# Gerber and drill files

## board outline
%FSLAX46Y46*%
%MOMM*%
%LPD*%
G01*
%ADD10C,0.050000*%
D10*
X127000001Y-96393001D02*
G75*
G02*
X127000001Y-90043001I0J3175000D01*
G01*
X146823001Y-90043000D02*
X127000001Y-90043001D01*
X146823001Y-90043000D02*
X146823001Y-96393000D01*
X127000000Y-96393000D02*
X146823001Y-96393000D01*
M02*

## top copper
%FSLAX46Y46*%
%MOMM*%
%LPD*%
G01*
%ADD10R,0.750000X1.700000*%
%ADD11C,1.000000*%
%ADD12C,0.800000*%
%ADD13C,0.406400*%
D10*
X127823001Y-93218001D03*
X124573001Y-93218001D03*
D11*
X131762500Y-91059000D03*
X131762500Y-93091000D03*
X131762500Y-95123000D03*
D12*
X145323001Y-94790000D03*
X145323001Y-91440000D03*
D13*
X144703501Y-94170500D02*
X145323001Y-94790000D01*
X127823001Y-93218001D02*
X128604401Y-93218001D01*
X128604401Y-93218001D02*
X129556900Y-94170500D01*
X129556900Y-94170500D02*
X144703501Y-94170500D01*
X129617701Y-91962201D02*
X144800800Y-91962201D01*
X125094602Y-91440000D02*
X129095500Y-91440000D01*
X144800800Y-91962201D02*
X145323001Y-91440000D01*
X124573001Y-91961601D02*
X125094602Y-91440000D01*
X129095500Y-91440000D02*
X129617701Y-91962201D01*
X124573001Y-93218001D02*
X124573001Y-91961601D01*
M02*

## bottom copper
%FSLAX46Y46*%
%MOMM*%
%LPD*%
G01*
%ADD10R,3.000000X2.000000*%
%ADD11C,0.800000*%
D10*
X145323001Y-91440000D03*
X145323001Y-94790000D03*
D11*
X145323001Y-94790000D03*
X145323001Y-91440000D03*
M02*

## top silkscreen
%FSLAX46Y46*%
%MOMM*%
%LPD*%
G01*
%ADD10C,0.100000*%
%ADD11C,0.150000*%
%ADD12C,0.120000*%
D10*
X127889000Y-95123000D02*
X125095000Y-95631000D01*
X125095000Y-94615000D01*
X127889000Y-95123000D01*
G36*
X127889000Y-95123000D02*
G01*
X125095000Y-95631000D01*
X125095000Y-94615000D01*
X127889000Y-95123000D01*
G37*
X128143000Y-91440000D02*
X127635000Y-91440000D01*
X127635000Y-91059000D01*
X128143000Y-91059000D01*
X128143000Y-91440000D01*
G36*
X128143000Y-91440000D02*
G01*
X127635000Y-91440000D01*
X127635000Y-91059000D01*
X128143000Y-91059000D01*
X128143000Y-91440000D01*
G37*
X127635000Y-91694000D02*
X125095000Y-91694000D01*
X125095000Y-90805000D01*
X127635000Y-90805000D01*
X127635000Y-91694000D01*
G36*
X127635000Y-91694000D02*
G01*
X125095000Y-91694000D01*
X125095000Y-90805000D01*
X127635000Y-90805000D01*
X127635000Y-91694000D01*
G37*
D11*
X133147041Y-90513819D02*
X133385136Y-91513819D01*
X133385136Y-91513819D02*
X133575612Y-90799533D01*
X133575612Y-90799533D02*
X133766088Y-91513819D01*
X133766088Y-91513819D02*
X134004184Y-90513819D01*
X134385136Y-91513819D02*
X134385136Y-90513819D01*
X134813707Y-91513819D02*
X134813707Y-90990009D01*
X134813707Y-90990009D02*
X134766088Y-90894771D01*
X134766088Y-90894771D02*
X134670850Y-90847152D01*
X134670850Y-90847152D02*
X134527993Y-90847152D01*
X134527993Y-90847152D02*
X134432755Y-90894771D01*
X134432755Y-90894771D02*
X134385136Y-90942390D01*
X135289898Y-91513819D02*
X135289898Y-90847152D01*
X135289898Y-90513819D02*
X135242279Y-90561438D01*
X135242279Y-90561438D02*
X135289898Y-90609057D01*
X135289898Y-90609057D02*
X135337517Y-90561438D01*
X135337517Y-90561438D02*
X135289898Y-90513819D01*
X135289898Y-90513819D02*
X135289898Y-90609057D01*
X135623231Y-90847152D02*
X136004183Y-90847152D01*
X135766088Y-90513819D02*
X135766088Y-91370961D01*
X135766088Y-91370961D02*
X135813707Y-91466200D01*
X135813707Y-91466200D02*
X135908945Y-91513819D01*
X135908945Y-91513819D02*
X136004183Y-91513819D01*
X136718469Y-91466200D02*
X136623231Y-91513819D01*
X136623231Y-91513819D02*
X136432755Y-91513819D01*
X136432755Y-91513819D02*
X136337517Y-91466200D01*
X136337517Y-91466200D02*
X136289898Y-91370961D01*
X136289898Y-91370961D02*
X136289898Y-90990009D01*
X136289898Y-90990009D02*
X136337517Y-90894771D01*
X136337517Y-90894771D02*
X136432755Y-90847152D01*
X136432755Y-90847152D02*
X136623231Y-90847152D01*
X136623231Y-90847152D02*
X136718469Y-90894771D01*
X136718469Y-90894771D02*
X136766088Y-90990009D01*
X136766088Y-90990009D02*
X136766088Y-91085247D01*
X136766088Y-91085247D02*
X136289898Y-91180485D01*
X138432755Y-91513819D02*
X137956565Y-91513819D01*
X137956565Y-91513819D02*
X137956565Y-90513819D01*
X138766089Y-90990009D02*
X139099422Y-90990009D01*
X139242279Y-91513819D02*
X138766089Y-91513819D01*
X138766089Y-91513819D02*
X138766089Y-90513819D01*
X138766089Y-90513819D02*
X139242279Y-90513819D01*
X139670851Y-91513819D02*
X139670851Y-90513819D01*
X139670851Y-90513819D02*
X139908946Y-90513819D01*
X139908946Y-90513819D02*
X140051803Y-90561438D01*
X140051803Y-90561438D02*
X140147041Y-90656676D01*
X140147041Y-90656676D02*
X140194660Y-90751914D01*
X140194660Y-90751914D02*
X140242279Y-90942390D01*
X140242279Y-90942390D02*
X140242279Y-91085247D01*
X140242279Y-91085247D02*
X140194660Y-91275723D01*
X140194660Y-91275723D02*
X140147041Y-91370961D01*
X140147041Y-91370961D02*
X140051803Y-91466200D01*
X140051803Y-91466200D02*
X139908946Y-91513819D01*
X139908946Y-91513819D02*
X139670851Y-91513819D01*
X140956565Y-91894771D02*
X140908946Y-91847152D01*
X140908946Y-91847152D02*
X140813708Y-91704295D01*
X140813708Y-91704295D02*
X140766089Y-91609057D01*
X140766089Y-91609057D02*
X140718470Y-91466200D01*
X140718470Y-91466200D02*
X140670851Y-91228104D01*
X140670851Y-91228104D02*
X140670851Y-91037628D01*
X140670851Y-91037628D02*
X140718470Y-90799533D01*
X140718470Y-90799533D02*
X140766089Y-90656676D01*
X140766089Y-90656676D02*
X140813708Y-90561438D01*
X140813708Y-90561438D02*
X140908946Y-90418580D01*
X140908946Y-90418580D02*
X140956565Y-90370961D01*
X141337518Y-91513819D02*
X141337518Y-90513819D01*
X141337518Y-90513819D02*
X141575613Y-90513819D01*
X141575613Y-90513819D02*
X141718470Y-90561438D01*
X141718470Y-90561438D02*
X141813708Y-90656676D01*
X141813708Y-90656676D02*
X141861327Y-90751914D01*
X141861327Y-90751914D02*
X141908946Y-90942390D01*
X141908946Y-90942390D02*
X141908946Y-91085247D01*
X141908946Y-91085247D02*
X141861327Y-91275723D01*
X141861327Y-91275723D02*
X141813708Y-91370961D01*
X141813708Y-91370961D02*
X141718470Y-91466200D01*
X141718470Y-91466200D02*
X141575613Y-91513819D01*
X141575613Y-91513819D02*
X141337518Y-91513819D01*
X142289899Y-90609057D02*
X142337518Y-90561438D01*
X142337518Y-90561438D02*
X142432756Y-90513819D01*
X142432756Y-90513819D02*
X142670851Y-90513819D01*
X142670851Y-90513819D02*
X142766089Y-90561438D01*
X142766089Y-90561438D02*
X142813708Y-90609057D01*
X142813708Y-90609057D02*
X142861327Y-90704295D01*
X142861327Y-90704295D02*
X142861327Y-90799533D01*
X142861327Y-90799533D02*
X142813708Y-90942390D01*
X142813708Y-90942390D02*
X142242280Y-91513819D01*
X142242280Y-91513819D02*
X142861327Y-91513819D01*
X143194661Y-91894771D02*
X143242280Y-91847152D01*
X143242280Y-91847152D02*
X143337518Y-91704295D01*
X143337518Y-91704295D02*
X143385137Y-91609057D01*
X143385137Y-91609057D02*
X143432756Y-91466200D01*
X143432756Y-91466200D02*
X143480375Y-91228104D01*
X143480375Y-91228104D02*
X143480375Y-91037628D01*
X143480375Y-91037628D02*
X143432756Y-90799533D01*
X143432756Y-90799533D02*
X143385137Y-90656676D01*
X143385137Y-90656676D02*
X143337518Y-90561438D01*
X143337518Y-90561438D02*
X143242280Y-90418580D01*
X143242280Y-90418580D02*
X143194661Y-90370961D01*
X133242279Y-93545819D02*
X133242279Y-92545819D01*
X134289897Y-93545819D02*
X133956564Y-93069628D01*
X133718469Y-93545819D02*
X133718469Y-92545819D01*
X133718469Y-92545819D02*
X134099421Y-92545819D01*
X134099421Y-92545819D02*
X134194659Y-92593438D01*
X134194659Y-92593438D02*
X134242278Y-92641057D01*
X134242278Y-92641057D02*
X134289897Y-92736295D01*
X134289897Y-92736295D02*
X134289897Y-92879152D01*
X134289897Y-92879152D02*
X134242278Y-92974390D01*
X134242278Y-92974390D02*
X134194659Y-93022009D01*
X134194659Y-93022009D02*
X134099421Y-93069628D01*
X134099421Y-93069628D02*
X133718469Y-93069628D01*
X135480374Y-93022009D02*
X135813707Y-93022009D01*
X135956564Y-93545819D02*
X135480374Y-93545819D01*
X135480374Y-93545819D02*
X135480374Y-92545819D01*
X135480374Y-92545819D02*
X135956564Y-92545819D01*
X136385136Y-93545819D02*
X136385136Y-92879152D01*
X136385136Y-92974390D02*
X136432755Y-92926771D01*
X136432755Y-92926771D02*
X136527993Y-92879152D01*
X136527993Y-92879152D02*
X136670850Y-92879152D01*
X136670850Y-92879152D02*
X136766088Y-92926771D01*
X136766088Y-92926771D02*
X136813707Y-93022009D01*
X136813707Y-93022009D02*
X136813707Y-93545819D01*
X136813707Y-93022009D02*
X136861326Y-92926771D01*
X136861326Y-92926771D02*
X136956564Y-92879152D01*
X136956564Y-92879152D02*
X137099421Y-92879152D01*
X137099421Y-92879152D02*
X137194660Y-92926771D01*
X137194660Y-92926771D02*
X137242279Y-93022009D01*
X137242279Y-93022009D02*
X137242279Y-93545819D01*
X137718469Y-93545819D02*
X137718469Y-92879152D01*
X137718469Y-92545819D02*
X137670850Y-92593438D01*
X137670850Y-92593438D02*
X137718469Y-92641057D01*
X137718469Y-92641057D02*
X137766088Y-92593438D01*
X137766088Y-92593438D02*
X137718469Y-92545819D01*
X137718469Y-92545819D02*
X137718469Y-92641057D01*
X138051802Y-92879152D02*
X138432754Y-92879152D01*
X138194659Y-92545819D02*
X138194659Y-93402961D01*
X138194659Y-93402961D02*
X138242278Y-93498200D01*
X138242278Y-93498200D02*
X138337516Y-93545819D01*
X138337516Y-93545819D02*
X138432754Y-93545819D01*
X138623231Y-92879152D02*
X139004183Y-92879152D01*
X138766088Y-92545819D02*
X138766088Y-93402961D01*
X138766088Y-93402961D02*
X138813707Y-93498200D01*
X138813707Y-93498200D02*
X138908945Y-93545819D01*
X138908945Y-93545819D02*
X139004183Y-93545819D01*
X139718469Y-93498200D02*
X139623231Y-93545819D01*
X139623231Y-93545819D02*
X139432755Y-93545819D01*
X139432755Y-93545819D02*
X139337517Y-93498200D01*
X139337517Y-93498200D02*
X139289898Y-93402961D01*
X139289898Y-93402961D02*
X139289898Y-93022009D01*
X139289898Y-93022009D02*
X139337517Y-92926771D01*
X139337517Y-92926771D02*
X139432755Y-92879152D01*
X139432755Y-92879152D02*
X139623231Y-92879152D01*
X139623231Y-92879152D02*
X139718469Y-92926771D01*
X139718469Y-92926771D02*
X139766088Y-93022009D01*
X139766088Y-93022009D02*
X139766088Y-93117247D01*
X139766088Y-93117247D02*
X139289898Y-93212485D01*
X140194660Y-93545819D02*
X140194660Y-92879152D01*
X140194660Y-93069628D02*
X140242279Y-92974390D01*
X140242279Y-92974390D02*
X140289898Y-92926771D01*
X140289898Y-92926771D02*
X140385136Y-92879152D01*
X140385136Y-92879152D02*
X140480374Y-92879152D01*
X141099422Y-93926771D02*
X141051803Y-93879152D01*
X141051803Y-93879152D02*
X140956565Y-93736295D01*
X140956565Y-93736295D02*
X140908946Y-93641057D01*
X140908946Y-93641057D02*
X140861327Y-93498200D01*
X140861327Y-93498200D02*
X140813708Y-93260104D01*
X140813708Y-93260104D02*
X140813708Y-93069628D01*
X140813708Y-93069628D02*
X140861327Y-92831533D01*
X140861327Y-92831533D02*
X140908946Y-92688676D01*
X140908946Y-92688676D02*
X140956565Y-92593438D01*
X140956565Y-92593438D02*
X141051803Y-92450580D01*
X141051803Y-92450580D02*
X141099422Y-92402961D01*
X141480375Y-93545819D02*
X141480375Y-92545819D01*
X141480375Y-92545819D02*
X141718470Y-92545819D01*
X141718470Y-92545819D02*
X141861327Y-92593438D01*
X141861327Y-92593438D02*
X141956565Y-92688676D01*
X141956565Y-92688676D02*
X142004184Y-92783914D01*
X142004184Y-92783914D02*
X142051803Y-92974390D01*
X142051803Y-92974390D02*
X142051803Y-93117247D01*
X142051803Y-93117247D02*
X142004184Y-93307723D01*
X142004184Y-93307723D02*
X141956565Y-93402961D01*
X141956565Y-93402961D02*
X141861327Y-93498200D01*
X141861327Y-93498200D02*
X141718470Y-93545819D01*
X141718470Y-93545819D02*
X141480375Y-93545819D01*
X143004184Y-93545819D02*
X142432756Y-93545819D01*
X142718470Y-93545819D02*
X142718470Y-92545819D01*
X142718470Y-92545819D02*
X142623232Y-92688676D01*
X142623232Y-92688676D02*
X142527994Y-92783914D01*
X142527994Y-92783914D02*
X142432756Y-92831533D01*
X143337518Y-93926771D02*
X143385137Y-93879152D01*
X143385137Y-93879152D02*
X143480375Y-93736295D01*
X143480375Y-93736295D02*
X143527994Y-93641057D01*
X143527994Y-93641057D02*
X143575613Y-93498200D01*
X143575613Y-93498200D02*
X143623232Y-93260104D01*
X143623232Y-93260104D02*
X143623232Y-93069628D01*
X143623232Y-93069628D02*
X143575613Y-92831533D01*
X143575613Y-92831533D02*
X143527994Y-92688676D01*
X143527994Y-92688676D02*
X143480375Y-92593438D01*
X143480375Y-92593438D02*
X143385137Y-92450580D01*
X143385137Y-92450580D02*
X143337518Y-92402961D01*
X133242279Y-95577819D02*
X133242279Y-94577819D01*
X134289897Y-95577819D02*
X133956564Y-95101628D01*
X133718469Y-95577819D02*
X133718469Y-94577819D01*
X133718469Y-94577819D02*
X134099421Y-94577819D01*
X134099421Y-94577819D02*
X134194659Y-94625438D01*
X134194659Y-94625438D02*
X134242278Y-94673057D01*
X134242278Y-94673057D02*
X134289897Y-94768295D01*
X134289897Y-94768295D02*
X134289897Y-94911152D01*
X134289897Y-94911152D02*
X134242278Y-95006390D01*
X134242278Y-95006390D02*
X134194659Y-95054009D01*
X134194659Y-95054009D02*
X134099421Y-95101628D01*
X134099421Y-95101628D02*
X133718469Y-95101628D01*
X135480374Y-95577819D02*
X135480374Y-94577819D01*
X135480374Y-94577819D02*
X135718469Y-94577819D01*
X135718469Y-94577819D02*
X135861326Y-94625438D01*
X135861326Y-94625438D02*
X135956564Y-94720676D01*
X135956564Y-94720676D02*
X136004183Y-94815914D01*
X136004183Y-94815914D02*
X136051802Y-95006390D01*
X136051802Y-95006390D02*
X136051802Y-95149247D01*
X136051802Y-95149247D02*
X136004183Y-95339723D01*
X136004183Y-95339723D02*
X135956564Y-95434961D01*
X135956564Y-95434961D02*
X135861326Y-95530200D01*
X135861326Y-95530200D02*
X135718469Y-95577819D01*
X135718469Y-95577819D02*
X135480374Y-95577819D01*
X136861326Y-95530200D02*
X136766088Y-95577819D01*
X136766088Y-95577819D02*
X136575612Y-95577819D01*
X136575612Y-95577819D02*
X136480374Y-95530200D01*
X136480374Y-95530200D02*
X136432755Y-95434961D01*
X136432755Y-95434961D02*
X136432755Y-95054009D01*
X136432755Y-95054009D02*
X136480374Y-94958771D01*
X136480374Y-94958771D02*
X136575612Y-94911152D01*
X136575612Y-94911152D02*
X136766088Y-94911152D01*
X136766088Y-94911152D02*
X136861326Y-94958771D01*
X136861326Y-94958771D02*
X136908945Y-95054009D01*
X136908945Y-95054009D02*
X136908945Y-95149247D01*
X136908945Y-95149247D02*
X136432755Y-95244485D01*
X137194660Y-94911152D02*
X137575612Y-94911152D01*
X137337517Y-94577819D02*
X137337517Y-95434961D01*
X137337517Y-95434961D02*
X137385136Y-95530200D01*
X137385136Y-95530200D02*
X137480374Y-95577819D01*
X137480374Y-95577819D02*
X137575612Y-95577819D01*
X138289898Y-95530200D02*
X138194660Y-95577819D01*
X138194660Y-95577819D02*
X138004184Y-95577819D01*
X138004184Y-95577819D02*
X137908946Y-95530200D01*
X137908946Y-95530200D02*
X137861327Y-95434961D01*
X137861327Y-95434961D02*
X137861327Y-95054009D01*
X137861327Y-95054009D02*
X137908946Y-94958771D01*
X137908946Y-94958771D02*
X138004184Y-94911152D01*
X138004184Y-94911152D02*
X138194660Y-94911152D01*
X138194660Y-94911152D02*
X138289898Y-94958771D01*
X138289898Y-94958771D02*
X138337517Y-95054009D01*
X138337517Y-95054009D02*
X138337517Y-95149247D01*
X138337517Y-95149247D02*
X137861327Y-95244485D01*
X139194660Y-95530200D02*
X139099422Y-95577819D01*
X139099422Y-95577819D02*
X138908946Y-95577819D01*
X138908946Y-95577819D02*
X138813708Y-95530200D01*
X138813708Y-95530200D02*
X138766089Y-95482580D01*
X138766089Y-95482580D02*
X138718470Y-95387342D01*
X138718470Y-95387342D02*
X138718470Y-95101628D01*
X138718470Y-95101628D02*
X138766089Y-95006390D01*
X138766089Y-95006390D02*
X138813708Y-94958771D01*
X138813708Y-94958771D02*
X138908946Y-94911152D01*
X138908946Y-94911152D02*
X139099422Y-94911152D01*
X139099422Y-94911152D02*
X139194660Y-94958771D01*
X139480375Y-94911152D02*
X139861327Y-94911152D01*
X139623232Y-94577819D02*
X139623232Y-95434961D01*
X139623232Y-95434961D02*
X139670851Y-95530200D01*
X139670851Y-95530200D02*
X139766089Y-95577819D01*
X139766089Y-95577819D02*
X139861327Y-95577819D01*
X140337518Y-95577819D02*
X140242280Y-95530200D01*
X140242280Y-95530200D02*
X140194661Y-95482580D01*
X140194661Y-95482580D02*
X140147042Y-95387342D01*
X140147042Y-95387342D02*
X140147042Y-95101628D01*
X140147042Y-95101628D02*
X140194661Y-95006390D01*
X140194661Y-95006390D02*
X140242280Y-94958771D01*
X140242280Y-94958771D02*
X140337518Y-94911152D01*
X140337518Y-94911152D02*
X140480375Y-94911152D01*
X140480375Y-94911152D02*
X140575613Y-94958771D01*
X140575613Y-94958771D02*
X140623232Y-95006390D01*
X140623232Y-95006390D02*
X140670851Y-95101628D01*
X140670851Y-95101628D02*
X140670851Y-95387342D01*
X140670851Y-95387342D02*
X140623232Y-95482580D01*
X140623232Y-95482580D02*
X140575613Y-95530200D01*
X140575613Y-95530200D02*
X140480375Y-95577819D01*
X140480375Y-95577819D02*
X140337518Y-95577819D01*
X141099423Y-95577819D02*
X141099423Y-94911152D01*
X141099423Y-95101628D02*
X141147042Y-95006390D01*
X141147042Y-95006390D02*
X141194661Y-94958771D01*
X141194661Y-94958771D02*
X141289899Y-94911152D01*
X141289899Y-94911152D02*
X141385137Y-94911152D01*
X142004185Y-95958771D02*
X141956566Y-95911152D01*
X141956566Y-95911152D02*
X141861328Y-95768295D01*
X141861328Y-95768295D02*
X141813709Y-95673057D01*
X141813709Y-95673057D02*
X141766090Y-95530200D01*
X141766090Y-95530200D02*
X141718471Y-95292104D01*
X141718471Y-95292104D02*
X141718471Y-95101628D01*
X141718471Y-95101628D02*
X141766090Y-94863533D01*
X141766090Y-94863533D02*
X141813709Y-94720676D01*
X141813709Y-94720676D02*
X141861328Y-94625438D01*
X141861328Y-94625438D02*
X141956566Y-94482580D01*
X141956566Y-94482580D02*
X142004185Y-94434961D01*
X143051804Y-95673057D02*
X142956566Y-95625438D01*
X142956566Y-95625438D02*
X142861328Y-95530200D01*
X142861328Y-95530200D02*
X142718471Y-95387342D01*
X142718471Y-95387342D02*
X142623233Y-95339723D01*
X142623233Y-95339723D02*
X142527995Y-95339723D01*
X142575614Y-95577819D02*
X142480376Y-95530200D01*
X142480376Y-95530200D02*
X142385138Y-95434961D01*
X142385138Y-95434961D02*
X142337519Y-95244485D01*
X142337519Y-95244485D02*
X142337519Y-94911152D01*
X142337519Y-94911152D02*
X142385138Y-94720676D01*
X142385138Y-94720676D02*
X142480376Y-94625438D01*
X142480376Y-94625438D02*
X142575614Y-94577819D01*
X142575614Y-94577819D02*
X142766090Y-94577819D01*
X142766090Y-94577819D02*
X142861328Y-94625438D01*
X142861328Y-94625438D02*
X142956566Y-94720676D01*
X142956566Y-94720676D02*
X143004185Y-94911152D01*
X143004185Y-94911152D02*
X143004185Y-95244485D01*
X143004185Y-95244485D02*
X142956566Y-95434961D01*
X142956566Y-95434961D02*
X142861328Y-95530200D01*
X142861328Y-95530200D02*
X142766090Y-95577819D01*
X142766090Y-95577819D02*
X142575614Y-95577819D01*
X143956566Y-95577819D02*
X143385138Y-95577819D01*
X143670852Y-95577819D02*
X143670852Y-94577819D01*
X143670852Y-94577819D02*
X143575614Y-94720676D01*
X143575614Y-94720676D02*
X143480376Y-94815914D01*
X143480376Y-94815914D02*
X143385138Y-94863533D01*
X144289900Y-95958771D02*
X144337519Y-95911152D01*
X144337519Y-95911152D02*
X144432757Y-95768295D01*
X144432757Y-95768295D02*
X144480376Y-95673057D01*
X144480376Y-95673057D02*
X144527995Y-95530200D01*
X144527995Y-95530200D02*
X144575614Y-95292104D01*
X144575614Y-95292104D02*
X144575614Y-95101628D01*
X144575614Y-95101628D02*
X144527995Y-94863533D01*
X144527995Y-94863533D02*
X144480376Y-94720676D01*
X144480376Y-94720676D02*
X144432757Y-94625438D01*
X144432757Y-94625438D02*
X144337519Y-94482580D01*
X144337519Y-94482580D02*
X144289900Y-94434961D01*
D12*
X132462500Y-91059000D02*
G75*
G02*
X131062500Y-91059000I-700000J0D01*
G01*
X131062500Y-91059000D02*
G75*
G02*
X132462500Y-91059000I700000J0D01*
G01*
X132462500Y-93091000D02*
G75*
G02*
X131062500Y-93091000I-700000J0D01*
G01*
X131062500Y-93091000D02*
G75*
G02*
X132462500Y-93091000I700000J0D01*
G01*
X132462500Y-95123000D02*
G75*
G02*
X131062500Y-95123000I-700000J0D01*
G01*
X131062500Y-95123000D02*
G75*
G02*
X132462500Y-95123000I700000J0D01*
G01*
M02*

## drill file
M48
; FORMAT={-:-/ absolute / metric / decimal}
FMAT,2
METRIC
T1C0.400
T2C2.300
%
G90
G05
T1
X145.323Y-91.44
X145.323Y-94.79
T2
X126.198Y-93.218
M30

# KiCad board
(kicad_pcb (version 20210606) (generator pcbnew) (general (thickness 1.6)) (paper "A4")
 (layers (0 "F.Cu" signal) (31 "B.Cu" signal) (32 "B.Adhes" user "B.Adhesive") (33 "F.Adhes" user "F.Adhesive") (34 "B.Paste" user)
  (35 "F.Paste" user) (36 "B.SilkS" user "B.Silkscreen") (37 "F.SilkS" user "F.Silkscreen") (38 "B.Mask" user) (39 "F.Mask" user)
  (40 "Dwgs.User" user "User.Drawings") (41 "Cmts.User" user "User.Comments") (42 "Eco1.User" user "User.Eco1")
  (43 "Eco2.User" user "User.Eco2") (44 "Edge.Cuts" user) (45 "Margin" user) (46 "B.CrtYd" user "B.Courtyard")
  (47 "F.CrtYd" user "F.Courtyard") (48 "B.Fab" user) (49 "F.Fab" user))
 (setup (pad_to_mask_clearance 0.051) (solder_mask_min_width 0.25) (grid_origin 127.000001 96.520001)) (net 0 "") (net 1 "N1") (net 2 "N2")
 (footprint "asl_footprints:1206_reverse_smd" (layer "F.Cu") (at 126.198001 93.218001 180)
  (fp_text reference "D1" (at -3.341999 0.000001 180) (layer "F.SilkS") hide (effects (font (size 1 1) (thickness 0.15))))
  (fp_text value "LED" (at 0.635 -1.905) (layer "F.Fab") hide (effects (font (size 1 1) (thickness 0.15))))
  (pad "" np_thru_hole circle locked (at 0 0 270) (size 2.3 2.3) (drill 2.3) (layers *.Cu *.Mask))
  (pad "1" smd rect locked (at -1.625 0 270) (size 1.7 0.75) (layers "F.Cu" "F.Paste" "F.Mask") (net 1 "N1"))
  (pad "2" smd rect locked (at 1.625 0 270) (size 1.7 0.75) (layers "F.Cu" "F.Paste" "F.Mask") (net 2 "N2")))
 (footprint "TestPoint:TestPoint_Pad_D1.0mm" (layer "F.Cu") (at 131.7625 91.059)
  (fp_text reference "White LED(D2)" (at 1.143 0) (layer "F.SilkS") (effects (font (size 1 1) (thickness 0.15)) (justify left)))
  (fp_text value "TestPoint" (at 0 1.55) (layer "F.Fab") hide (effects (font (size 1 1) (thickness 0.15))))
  (fp_circle (center 0 0) (end 0 0.7) (layer "F.SilkS") (width 0.12) (fill none))
  (pad "1" smd circle locked (at 0 0) (size 1 1) (layers "F.Cu" "F.Mask")))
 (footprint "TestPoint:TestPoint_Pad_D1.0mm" (layer "F.Cu") (at 131.7625 93.091)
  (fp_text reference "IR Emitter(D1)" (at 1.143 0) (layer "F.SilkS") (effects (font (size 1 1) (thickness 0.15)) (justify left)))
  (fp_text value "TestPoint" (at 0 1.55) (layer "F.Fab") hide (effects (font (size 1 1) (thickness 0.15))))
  (fp_circle (center 0 0) (end 0 0.7) (layer "F.SilkS") (width 0.12) (fill none))
  (pad "1" smd circle locked (at 0 0) (size 1 1) (layers "F.Cu" "F.Mask")))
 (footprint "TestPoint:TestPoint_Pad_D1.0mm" (layer "F.Cu") (at 131.7625 95.123)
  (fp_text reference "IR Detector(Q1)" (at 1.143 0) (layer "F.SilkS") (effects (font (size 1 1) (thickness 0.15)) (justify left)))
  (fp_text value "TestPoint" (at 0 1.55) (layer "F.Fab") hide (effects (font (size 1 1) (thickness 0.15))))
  (fp_circle (center 0 0) (end 0 0.7) (layer "F.SilkS") (width 0.12) (fill none))
  (pad "1" smd circle locked (at 0 0) (size 1 1) (layers "F.Cu" "F.Mask")))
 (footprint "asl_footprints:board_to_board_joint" (layer "B.Cu") (at 146.823001 93.115 -90)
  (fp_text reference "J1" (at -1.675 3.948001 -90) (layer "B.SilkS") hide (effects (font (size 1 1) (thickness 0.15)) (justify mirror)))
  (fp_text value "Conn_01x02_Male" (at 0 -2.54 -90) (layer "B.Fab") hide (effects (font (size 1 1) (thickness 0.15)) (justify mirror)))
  (pad "1" smd rect locked (at -1.675 1.5 270) (size 2 3) (layers "B.Cu" "B.Paste" "B.Mask") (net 2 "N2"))
  (pad "2" smd rect locked (at 1.675 1.5 270) (size 2 3) (layers "B.Cu" "B.Paste" "B.Mask") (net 1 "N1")))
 (gr_poly (pts (xy 127.889 95.123) (xy 125.095 95.631) (xy 125.095 94.615)) (layer "F.SilkS") (width 0.1) (fill solid))
 (gr_poly (pts (xy 128.143 91.44) (xy 127.635 91.44) (xy 127.635 91.059) (xy 128.143 91.059)) (layer "F.SilkS") (width 0.1) (fill solid))
 (gr_poly (pts (xy 127.635 91.694) (xy 125.095 91.694) (xy 125.095 90.805) (xy 127.635 90.805)) (layer "F.SilkS") (width 0.1) (fill solid))
 (gr_arc (start 127.000001 93.218001) (end 127.000001 90.043001) (angle -180) (layer "Edge.Cuts") (width 0.05))
 (gr_line (start 146.823001 90.043) (end 127.000001 90.043001) (layer "Edge.Cuts") (width 0.05))
 (gr_line (start 146.823001 90.043) (end 146.823001 96.393) (layer "Edge.Cuts") (width 0.05))
 (gr_line (start 127 96.393) (end 146.823001 96.393) (layer "Edge.Cuts") (width 0.05))
 (segment (start 144.703501 94.1705) (end 145.323001 94.79) (width 0.4064) (layer "F.Cu") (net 1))
 (segment (start 127.823001 93.218001) (end 128.604401 93.218001) (width 0.4064) (layer "F.Cu") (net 1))
 (segment (start 128.604401 93.218001) (end 129.5569 94.1705) (width 0.4064) (layer "F.Cu") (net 1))
 (segment (start 129.5569 94.1705) (end 144.703501 94.1705) (width 0.4064) (layer "F.Cu") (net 1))
 (via (at 145.323001 94.79) (size 0.8) (drill 0.4) (layers "F.Cu" "B.Cu") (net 1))
 (segment (start 129.617701 91.962201) (end 144.8008 91.962201) (width 0.4064) (layer "F.Cu") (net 2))
 (segment (start 125.094602 91.44) (end 129.0955 91.44) (width 0.4064) (layer "F.Cu") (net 2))
 (segment (start 144.8008 91.962201) (end 145.323001 91.44) (width 0.4064) (layer "F.Cu") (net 2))
 (segment (start 124.573001 91.961601) (end 125.094602 91.44) (width 0.4064) (layer "F.Cu") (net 2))
 (segment (start 129.0955 91.44) (end 129.617701 91.962201) (width 0.4064) (layer "F.Cu") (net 2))
 (segment (start 124.573001 93.218001) (end 124.573001 91.961601) (width 0.4064) (layer "F.Cu") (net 2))
 (via (at 145.323001 91.44) (size 0.8) (drill 0.4) (layers "F.Cu" "B.Cu") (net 2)))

